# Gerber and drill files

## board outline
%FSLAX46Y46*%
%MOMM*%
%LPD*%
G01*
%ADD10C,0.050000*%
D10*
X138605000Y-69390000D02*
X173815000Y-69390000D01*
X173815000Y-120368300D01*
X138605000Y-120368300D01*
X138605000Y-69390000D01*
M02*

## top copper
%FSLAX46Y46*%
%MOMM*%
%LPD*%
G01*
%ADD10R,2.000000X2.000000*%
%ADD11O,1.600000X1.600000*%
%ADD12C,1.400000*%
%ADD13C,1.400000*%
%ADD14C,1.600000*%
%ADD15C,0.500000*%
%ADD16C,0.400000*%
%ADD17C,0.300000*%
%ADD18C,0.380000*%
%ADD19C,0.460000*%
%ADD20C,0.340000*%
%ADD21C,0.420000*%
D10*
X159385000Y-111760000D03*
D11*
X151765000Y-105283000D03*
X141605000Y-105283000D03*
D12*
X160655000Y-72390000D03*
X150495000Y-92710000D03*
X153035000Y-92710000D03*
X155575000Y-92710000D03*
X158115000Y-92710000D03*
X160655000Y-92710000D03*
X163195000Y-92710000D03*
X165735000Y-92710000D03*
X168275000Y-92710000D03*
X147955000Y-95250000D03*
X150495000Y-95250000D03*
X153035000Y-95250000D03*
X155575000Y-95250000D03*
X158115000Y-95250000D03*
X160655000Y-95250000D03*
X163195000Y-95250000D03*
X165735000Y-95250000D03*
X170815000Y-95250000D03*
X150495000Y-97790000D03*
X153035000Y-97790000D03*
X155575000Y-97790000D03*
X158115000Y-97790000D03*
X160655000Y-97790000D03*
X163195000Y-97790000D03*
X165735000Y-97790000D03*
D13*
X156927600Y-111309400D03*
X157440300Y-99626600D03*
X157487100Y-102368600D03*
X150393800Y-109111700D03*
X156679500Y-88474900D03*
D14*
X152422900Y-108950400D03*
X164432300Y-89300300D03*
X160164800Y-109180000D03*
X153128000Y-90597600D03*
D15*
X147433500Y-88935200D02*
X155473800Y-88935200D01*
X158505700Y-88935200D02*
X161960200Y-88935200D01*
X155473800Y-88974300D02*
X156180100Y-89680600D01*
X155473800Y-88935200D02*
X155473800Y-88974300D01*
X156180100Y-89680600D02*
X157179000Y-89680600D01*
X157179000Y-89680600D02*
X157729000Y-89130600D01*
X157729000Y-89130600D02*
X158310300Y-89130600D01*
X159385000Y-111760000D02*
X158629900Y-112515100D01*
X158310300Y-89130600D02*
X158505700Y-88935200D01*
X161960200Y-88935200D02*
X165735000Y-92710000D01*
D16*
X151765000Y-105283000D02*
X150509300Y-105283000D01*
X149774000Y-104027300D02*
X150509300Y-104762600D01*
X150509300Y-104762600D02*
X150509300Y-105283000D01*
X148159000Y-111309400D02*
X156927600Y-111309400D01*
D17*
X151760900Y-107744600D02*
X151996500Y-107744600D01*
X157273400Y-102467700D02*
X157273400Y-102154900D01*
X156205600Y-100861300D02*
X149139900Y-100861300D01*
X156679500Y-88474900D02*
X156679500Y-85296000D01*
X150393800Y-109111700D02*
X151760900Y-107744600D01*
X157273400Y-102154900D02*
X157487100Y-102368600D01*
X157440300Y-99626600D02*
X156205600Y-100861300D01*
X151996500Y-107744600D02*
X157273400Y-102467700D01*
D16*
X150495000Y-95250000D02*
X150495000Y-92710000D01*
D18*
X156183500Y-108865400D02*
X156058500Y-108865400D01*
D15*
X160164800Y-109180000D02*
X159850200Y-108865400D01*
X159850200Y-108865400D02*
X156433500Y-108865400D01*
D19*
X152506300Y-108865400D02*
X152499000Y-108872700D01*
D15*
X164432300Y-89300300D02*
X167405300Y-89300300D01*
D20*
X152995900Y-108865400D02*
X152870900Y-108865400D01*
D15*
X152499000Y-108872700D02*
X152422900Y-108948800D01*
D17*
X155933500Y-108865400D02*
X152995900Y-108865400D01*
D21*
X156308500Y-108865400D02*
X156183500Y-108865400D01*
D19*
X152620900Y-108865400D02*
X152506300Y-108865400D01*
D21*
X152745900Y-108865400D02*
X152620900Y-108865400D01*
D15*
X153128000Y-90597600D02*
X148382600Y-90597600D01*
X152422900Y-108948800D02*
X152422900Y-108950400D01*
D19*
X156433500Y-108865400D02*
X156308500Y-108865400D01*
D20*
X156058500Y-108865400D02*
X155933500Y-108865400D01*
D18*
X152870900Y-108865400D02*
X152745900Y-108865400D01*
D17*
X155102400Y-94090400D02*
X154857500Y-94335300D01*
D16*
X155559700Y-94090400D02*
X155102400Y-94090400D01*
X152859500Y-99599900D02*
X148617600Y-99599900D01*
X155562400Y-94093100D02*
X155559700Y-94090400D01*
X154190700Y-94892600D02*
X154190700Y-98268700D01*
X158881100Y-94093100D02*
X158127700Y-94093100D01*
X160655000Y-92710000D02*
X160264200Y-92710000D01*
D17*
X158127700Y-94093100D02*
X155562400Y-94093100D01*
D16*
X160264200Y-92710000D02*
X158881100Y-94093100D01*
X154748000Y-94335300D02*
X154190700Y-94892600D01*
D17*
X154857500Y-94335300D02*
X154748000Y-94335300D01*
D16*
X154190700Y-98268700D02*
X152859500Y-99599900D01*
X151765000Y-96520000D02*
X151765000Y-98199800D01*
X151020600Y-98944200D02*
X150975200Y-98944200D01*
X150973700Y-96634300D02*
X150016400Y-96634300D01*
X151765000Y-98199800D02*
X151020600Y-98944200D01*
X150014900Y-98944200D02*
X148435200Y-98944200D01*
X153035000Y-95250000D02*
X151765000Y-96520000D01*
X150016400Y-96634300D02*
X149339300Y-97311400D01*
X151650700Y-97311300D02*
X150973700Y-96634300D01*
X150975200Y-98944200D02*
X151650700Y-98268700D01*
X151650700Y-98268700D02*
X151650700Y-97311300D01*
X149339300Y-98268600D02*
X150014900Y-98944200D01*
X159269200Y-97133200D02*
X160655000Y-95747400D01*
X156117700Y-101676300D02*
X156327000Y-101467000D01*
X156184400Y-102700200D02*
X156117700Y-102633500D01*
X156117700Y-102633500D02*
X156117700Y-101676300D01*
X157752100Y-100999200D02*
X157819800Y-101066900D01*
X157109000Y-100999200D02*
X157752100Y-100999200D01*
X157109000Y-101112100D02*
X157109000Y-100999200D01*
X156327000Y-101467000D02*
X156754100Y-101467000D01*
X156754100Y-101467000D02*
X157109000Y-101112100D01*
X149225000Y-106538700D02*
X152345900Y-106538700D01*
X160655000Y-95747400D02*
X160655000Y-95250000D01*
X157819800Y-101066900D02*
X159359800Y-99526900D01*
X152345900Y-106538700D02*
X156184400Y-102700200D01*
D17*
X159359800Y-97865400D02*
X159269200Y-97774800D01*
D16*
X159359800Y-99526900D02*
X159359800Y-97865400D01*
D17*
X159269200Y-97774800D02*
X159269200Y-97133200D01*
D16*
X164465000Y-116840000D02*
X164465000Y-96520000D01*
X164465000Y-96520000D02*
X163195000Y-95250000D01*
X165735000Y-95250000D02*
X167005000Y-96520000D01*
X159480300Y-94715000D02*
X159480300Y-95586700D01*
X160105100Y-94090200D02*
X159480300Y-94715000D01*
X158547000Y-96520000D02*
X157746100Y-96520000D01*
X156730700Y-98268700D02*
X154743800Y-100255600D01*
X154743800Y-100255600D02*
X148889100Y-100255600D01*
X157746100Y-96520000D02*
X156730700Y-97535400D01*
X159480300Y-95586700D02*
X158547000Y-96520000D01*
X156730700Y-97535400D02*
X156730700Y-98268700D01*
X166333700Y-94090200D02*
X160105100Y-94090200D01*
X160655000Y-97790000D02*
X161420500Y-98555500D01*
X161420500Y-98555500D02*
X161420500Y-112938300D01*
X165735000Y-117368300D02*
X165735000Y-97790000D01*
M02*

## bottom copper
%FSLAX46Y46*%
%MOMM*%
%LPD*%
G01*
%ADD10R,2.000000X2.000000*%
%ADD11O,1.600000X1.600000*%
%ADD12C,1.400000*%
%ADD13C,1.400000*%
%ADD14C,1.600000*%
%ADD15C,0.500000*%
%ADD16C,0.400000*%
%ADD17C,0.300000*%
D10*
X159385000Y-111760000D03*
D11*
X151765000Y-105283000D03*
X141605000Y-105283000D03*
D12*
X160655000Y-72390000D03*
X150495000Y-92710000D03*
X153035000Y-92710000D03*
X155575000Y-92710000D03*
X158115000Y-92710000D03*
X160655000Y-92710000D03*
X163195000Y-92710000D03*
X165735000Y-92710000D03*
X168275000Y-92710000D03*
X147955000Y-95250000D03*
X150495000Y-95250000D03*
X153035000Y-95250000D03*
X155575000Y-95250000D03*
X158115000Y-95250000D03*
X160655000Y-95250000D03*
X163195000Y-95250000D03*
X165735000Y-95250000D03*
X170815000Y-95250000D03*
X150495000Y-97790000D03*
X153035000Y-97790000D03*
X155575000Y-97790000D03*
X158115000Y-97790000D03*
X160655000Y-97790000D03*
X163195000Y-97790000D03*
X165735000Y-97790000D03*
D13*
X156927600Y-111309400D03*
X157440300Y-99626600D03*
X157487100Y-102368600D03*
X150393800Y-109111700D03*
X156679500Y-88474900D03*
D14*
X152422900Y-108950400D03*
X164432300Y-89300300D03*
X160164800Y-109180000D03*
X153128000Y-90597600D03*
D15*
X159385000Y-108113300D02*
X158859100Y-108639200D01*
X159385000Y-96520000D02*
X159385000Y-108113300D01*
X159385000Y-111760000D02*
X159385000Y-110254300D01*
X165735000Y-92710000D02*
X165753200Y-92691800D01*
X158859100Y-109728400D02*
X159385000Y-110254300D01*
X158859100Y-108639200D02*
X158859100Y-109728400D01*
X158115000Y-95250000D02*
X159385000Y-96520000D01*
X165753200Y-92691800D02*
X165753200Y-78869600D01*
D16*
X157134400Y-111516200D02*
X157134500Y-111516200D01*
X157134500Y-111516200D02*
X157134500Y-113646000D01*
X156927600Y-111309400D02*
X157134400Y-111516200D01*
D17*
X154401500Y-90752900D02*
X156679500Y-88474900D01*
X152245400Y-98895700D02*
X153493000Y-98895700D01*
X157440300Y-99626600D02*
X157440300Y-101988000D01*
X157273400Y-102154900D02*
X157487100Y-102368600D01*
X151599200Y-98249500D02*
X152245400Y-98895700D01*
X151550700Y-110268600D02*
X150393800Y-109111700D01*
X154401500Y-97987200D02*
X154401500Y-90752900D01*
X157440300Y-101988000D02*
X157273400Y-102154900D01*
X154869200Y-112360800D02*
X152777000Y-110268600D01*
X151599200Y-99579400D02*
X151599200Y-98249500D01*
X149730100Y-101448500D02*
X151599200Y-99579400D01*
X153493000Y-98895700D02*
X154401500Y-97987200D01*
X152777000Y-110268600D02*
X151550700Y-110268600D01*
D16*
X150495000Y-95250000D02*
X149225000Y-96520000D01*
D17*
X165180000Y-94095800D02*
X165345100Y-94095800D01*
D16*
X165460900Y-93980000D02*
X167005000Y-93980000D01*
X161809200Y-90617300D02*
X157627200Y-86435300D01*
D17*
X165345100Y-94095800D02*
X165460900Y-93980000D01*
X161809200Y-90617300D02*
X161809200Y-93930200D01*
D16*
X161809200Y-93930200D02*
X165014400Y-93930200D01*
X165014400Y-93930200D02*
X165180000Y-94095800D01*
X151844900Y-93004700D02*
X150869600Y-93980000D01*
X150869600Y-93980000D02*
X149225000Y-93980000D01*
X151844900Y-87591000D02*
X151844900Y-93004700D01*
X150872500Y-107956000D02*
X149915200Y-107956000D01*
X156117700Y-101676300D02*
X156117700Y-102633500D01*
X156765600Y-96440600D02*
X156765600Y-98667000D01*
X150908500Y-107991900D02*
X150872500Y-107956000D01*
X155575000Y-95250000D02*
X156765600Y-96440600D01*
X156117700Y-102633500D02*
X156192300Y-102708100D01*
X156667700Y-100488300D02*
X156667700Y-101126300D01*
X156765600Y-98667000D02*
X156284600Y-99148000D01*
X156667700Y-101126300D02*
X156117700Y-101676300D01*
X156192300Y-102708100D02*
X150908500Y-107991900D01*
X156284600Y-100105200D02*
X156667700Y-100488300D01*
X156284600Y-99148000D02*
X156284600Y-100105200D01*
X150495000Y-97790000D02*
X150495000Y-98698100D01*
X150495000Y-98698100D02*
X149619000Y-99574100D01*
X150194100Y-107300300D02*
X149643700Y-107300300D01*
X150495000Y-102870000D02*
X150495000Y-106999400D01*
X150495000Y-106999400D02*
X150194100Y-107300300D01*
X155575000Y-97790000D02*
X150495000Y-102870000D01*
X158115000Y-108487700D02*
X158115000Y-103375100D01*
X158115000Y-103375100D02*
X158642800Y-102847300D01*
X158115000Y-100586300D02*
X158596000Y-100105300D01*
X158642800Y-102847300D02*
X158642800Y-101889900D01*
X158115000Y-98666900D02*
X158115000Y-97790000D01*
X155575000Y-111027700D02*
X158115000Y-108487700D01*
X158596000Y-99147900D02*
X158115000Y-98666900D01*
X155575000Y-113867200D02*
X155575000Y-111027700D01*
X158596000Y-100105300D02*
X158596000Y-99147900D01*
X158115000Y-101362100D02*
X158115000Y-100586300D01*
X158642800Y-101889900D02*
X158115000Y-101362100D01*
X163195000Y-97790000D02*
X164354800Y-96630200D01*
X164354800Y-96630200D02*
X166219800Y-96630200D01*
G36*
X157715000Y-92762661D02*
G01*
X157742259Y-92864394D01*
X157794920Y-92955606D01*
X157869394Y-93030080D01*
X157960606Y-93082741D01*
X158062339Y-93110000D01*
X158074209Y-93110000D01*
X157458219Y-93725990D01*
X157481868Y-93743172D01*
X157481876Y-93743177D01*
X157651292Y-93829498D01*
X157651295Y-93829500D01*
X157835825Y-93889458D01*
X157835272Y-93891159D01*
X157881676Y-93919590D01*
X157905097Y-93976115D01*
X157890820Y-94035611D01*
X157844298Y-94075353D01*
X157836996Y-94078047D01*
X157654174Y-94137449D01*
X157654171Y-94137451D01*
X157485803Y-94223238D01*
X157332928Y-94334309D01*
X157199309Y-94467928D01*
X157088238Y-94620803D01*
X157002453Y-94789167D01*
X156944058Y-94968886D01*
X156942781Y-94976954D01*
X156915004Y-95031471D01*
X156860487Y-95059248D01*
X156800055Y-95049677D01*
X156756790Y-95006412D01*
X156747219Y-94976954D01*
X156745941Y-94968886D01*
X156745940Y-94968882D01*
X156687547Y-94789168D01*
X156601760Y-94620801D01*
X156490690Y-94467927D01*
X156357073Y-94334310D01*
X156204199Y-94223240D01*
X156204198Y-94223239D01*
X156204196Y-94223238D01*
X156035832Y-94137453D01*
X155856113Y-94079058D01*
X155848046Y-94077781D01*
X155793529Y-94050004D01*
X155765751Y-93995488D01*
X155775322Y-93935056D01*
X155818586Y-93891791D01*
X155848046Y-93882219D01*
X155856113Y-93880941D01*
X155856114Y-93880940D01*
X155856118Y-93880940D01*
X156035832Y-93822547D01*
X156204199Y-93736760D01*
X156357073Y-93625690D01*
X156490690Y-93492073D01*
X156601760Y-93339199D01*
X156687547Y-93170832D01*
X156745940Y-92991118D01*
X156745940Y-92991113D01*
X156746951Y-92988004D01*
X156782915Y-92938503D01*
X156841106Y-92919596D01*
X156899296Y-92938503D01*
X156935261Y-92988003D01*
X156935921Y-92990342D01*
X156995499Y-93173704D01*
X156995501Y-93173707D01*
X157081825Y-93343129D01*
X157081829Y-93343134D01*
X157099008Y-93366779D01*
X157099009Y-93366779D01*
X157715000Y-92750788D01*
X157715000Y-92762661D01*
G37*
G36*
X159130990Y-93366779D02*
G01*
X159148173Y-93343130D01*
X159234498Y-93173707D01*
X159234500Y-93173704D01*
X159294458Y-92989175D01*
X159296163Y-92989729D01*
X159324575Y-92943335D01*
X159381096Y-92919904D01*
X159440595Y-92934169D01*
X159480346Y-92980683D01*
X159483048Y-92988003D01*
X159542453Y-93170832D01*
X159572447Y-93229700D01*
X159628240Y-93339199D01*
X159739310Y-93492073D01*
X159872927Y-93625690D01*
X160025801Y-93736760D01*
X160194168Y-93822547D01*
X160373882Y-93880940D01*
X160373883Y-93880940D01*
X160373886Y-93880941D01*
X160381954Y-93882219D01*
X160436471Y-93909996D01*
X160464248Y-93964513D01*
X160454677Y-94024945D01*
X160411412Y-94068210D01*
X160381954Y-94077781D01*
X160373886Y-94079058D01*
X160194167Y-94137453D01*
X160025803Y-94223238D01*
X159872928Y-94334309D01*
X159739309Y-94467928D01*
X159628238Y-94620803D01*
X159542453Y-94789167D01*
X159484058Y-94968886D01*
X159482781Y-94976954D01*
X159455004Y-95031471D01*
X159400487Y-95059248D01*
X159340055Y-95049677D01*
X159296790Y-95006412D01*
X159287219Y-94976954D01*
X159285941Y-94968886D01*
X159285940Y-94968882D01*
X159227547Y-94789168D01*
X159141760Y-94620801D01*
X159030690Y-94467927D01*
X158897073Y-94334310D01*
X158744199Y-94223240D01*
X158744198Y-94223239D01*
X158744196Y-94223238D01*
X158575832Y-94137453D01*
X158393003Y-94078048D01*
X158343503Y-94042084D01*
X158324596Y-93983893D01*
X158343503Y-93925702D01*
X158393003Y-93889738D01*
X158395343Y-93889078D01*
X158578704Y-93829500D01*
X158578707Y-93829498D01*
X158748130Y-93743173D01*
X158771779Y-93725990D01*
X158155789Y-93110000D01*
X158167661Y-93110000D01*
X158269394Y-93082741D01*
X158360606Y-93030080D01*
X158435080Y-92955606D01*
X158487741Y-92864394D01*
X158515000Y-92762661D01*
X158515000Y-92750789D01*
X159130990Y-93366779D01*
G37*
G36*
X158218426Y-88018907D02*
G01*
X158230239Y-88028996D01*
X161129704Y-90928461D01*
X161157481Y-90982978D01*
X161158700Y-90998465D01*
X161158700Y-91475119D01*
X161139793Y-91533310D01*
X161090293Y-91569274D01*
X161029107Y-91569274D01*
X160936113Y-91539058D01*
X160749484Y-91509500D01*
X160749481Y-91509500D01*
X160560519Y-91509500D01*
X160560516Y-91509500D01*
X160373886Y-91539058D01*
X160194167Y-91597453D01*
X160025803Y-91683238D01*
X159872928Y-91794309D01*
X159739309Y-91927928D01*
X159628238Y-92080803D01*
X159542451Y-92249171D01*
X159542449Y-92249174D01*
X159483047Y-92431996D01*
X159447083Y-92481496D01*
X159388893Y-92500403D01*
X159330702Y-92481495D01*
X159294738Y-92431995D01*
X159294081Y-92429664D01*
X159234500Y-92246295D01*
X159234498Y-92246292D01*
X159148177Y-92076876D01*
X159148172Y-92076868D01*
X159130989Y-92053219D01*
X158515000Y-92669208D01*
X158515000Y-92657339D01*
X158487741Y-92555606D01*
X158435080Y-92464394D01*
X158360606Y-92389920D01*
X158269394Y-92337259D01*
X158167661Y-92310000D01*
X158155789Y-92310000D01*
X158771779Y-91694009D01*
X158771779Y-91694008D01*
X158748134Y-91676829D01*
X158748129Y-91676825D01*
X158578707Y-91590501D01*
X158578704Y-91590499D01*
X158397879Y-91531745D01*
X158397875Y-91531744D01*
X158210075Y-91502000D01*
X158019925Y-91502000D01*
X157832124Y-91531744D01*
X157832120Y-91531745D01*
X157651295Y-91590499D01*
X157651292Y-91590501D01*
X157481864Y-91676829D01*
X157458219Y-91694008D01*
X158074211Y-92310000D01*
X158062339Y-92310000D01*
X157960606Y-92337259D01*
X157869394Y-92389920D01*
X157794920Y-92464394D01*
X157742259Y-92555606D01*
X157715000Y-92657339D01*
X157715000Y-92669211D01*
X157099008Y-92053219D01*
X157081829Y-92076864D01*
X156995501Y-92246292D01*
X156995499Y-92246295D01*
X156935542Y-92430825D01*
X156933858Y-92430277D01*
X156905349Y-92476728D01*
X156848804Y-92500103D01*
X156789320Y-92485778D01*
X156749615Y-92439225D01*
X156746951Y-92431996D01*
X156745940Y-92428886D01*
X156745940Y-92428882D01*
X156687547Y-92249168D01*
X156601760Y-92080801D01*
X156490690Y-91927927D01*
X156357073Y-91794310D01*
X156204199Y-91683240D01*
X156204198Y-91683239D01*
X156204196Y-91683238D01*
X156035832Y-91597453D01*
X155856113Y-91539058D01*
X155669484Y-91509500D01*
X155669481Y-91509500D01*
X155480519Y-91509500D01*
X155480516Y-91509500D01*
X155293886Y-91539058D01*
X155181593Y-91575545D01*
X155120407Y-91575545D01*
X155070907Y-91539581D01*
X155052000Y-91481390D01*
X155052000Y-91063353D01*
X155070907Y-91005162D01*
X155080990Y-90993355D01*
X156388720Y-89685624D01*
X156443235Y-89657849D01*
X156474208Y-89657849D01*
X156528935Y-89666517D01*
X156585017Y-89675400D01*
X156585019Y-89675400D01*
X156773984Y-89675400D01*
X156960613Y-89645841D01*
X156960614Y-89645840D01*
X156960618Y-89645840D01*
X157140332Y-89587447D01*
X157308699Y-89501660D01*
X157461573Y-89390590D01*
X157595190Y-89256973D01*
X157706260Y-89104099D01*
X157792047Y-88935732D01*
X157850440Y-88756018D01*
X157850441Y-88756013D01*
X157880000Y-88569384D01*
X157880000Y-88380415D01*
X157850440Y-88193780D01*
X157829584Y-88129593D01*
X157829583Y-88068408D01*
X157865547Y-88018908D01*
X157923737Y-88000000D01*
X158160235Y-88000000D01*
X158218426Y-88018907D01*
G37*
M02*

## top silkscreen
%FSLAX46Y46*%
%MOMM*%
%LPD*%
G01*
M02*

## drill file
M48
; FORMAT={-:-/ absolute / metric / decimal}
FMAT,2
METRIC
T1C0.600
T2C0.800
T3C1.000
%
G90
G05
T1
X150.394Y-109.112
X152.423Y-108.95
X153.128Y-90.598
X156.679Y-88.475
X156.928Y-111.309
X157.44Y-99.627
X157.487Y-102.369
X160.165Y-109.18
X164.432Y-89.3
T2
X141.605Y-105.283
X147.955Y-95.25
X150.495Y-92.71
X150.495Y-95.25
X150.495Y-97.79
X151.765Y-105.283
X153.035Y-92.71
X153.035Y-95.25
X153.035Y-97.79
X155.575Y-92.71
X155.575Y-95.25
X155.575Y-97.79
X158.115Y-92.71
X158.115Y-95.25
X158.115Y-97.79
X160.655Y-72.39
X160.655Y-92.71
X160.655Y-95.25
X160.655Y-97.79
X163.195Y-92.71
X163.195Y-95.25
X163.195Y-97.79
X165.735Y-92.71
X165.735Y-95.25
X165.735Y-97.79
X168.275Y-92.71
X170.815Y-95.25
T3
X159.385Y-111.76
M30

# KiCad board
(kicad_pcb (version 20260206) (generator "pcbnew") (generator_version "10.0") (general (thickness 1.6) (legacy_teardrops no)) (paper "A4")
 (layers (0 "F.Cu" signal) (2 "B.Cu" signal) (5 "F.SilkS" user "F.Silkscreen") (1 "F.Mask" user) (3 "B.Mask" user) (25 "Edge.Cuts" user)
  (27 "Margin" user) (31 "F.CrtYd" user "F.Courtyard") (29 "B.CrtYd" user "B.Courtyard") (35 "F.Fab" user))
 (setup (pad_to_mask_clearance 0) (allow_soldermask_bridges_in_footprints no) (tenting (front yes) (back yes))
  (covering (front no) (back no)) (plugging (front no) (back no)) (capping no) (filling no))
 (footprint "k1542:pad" (layer "F.Cu") (at 159.385 111.76)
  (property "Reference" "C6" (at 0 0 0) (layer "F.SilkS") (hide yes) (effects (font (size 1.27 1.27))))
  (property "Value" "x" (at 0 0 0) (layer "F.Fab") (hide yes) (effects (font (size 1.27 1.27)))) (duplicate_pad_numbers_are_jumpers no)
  (pad "1" thru_hole rect (at 0 0) (size 2 2) (drill 1) (layers "*.Cu" "*.Mask") (remove_unused_layers no) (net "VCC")))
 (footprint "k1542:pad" (layer "F.Cu") (at 151.765 105.283 90)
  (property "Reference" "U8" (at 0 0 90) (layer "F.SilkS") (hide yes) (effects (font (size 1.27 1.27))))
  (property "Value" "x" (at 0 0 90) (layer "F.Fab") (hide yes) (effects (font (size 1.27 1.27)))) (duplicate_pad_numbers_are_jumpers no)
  (pad "13" thru_hole oval (at 0 0 90) (size 1.6 1.6) (drill 0.8) (layers "*.Cu" "*.Mask") (remove_unused_layers no) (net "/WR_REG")))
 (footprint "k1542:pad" (layer "F.Cu") (at 141.605 105.283 90)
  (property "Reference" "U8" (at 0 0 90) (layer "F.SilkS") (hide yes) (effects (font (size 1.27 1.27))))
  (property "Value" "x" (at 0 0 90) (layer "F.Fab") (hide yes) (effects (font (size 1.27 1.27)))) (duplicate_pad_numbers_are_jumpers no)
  (pad "17" thru_hole oval (at 0 0 90) (size 1.6 1.6) (drill 0.8) (layers "*.Cu" "*.Mask") (remove_unused_layers no) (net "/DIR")))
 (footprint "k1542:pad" (layer "F.Cu") (at 160.655 72.39 180)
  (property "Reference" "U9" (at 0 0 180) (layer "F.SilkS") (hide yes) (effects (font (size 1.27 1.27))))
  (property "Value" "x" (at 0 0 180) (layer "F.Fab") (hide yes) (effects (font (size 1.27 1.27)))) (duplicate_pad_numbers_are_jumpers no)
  (pad "C8" thru_hole circle (at 0 0 180) (size 1.4 1.4) (drill 0.8) (layers "*.Cu" "*.Mask") (remove_unused_layers no) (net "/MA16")))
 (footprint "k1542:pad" (layer "F.Cu") (at 150.495 92.71 180)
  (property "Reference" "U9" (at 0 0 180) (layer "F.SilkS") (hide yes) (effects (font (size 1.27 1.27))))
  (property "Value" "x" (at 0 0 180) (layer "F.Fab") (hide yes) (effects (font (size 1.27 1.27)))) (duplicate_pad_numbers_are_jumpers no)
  (pad "L4" thru_hole circle (at 0 0 180) (size 1.4 1.4) (drill 0.8) (layers "*.Cu" "*.Mask") (remove_unused_layers no) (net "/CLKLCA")))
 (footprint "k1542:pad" (layer "F.Cu") (at 153.035 92.71 180)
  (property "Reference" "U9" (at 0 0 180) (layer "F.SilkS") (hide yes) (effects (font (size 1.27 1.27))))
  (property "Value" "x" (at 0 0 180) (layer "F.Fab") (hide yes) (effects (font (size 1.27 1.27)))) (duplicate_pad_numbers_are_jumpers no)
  (pad "L5" thru_hole circle (at 0 0 180) (size 1.4 1.4) (drill 0.8) (layers "*.Cu" "*.Mask") (remove_unused_layers no)
   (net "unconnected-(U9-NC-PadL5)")))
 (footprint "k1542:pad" (layer "F.Cu") (at 155.575 92.71 180)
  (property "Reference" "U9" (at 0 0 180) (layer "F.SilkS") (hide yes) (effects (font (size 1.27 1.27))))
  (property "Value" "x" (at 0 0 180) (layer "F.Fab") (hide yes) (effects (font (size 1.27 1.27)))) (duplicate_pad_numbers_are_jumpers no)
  (pad "L6" thru_hole circle (at 0 0 180) (size 1.4 1.4) (drill 0.8) (layers "*.Cu" "*.Mask") (remove_unused_layers no)
   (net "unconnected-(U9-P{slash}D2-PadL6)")))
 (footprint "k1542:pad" (layer "F.Cu") (at 158.115 92.71 180)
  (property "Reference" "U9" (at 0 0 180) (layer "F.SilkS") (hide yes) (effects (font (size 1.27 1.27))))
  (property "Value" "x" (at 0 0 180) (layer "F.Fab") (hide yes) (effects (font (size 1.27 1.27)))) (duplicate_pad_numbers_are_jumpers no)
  (pad "L7" thru_hole circle (at 0 0 180) (size 1.4 1.4) (drill 0.8) (layers "*.Cu" "*.Mask") (remove_unused_layers no) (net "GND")))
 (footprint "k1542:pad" (layer "F.Cu") (at 160.655 92.71 180)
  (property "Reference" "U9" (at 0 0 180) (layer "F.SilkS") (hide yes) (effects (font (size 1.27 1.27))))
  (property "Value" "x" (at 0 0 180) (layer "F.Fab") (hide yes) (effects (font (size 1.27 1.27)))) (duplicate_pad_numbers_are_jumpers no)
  (pad "L8" thru_hole circle (at 0 0 180) (size 1.4 1.4) (drill 0.8) (layers "*.Cu" "*.Mask") (remove_unused_layers no) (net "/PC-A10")))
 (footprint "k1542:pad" (layer "F.Cu") (at 163.195 92.71 180)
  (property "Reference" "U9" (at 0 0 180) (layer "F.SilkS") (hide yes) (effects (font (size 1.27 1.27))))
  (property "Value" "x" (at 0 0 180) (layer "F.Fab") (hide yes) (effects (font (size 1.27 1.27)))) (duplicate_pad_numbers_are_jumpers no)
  (pad "L9" thru_hole circle (at 0 0 180) (size 1.4 1.4) (drill 0.8) (layers "*.Cu" "*.Mask") (remove_unused_layers no)
   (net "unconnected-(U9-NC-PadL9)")))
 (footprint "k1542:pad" (layer "F.Cu") (at 165.735 92.71 180)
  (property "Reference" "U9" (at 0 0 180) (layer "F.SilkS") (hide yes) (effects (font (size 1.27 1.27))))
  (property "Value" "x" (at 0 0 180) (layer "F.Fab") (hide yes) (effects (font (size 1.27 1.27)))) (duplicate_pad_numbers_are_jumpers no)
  (pad "L10" thru_hole circle (at 0 0 180) (size 1.4 1.4) (drill 0.8) (layers "*.Cu" "*.Mask") (remove_unused_layers no) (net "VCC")))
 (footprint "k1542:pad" (layer "F.Cu") (at 168.275 92.71 180)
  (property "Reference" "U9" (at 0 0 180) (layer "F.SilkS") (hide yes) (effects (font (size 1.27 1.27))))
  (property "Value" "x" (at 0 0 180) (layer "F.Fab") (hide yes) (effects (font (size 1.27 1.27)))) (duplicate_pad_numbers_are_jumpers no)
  (pad "L11" thru_hole circle (at 0 0 180) (size 1.4 1.4) (drill 0.8) (layers "*.Cu" "*.Mask") (remove_unused_layers no) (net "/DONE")))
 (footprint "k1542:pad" (layer "F.Cu") (at 147.955 95.25 180)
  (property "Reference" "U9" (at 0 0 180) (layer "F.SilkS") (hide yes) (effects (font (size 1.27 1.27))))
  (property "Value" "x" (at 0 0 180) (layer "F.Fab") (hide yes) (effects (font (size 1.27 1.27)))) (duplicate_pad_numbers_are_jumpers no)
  (pad "M3" thru_hole circle (at 0 0 180) (size 1.4 1.4) (drill 0.8) (layers "*.Cu" "*.Mask") (remove_unused_layers no) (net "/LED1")))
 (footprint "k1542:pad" (layer "F.Cu") (at 150.495 95.25 180)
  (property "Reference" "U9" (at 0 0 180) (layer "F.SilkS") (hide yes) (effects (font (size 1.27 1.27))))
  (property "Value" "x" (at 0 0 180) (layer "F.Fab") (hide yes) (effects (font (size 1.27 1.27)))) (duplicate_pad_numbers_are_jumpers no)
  (pad "M4" thru_hole circle (at 0 0 180) (size 1.4 1.4) (drill 0.8) (layers "*.Cu" "*.Mask") (remove_unused_layers no) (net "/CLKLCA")))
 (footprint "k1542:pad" (layer "F.Cu") (at 153.035 95.25 180)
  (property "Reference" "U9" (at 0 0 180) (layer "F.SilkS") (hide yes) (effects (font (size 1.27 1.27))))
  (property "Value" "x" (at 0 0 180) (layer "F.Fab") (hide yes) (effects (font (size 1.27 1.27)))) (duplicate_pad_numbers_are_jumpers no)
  (pad "M5" thru_hole circle (at 0 0 180) (size 1.4 1.4) (drill 0.8) (layers "*.Cu" "*.Mask") (remove_unused_layers no) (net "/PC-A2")))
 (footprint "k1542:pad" (layer "F.Cu") (at 155.575 95.25 180)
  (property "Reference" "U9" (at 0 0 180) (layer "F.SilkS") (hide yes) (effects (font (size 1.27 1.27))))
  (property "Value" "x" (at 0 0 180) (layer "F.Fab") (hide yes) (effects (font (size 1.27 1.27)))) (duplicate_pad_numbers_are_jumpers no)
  (pad "M6" thru_hole circle (at 0 0 180) (size 1.4 1.4) (drill 0.8) (layers "*.Cu" "*.Mask") (remove_unused_layers no) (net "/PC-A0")))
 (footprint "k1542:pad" (layer "F.Cu") (at 158.115 95.25 180)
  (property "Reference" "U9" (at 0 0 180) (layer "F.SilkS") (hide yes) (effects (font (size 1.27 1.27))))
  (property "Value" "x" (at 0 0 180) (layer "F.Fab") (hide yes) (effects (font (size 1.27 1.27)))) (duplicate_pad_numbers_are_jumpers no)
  (pad "M7" thru_hole circle (at 0 0 180) (size 1.4 1.4) (drill 0.8) (layers "*.Cu" "*.Mask") (remove_unused_layers no) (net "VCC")))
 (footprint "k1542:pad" (layer "F.Cu") (at 160.655 95.25 180)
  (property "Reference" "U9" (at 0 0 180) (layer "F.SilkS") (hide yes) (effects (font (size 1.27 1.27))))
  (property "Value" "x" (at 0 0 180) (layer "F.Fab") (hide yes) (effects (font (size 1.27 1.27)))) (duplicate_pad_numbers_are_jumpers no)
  (pad "M8" thru_hole circle (at 0 0 180) (size 1.4 1.4) (drill 0.8) (layers "*.Cu" "*.Mask") (remove_unused_layers no) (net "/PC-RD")))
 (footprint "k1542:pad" (layer "F.Cu") (at 163.195 95.25 180)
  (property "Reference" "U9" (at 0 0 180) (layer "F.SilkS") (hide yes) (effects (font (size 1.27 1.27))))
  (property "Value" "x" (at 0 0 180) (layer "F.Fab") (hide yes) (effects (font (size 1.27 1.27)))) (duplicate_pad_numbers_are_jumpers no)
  (pad "M9" thru_hole circle (at 0 0 180) (size 1.4 1.4) (drill 0.8) (layers "*.Cu" "*.Mask") (remove_unused_layers no) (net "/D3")))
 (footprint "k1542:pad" (layer "F.Cu") (at 165.735 95.25 180)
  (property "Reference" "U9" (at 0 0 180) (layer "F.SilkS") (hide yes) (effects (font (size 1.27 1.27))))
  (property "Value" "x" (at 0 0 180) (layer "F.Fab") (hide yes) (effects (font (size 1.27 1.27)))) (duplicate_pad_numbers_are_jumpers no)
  (pad "M10" thru_hole circle (at 0 0 180) (size 1.4 1.4) (drill 0.8) (layers "*.Cu" "*.Mask") (remove_unused_layers no) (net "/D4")))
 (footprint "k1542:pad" (layer "F.Cu") (at 170.815 95.25 180)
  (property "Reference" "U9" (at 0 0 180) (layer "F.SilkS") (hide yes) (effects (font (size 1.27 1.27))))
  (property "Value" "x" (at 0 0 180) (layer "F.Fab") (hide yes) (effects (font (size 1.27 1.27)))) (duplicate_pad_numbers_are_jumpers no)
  (pad "M12" thru_hole circle (at 0 0 180) (size 1.4 1.4) (drill 0.8) (layers "*.Cu" "*.Mask") (remove_unused_layers no) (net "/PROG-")))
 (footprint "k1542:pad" (layer "F.Cu") (at 150.495 97.79 180)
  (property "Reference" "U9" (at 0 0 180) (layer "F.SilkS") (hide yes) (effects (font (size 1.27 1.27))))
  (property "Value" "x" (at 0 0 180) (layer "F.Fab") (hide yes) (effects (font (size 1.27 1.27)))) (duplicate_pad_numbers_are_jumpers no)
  (pad "N4" thru_hole circle (at 0 0 180) (size 1.4 1.4) (drill 0.8) (layers "*.Cu" "*.Mask") (remove_unused_layers no) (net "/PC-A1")))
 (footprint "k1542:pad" (layer "F.Cu") (at 153.035 97.79 180)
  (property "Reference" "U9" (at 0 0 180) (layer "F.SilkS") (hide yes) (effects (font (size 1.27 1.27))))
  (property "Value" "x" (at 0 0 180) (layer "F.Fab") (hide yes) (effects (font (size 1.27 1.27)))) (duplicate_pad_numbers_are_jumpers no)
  (pad "N5" thru_hole circle (at 0 0 180) (size 1.4 1.4) (drill 0.8) (layers "*.Cu" "*.Mask") (remove_unused_layers no)
   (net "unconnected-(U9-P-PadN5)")))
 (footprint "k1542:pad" (layer "F.Cu") (at 155.575 97.79 180)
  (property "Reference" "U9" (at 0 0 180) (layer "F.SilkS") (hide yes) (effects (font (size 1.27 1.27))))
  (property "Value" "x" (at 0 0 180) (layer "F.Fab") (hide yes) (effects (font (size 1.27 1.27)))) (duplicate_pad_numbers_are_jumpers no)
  (pad "N6" thru_hole circle (at 0 0 180) (size 1.4 1.4) (drill 0.8) (layers "*.Cu" "*.Mask") (remove_unused_layers no) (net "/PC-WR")))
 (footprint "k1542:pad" (layer "F.Cu") (at 158.115 97.79 180)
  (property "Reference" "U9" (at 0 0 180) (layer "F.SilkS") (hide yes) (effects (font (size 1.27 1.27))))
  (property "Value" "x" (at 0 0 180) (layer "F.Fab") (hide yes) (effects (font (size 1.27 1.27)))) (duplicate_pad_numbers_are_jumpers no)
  (pad "N7" thru_hole circle (at 0 0 180) (size 1.4 1.4) (drill 0.8) (layers "*.Cu" "*.Mask") (remove_unused_layers no) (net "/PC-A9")))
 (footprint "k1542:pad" (layer "F.Cu") (at 160.655 97.79 180)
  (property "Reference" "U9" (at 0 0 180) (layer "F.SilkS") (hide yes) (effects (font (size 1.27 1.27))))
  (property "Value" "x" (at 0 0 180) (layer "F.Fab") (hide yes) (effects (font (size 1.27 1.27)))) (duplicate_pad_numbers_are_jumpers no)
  (pad "N8" thru_hole circle (at 0 0 180) (size 1.4 1.4) (drill 0.8) (layers "*.Cu" "*.Mask") (remove_unused_layers no) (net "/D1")))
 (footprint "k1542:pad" (layer "F.Cu") (at 163.195 97.79 180)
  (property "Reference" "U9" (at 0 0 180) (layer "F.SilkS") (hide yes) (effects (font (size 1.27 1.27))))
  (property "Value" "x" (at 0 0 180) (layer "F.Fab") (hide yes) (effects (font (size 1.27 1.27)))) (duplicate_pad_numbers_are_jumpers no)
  (pad "N9" thru_hole circle (at 0 0 180) (size 1.4 1.4) (drill 0.8) (layers "*.Cu" "*.Mask") (remove_unused_layers no) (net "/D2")))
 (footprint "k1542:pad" (layer "F.Cu") (at 165.735 97.79 180)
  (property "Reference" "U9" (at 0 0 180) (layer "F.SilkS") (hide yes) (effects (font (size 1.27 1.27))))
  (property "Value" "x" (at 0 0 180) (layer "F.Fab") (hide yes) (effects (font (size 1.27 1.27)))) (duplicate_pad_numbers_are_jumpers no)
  (pad "N10" thru_hole circle (at 0 0 180) (size 1.4 1.4) (drill 0.8) (layers "*.Cu" "*.Mask") (remove_unused_layers no) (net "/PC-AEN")))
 (gr_rect (start 138.605 69.39) (end 173.815 120.3683) (stroke (width 0.05) (type default)) (fill no) (layer "Edge.Cuts"))
 (segment (start 147.4335 88.9352) (end 155.4738 88.9352) (width 0.5) (layer "F.Cu") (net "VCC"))
 (segment (start 158.5057 88.9352) (end 161.9602 88.9352) (width 0.5) (layer "F.Cu") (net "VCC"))
 (segment (start 155.4738 88.9743) (end 156.1801 89.6806) (width 0.5) (layer "F.Cu") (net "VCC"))
 (segment (start 155.4738 88.9352) (end 155.4738 88.9743) (width 0.5) (layer "F.Cu") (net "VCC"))
 (segment (start 156.1801 89.6806) (end 157.179 89.6806) (width 0.5) (layer "F.Cu") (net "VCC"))
 (segment (start 157.179 89.6806) (end 157.729 89.1306) (width 0.5) (layer "F.Cu") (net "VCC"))
 (segment (start 157.729 89.1306) (end 158.3103 89.1306) (width 0.5) (layer "F.Cu") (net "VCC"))
 (segment (start 159.385 111.76) (end 158.6299 112.5151) (width 0.5) (layer "F.Cu") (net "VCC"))
 (segment (start 158.3103 89.1306) (end 158.5057 88.9352) (width 0.5) (layer "F.Cu") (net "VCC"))
 (segment (start 161.9602 88.9352) (end 165.735 92.71) (width 0.5) (layer "F.Cu") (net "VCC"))
 (segment (start 159.385 108.1133) (end 158.8591 108.6392) (width 0.5) (layer "B.Cu") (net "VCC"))
 (segment (start 159.385 96.52) (end 159.385 108.1133) (width 0.5) (layer "B.Cu") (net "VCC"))
 (segment (start 159.385 111.76) (end 159.385 110.2543) (width 0.5) (layer "B.Cu") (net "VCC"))
 (segment (start 165.735 92.71) (end 165.7532 92.6918) (width 0.5) (layer "B.Cu") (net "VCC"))
 (segment (start 158.8591 109.7284) (end 159.385 110.2543) (width 0.5) (layer "B.Cu") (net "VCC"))
 (segment (start 158.8591 108.6392) (end 158.8591 109.7284) (width 0.5) (layer "B.Cu") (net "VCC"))
 (segment (start 158.115 95.25) (end 159.385 96.52) (width 0.5) (layer "B.Cu") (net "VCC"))
 (segment (start 165.7532 92.6918) (end 165.7532 78.8696) (width 0.5) (layer "B.Cu") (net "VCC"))
 (segment (start 151.765 105.283) (end 150.5093 105.283) (width 0.4) (layer "F.Cu") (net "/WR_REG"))
 (segment (start 149.774 104.0273) (end 150.5093 104.7626) (width 0.4) (layer "F.Cu") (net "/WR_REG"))
 (segment (start 150.5093 104.7626) (end 150.5093 105.283) (width 0.4) (layer "F.Cu") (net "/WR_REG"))
 (segment (start 148.159 111.3094) (end 156.9276 111.3094) (width 0.4) (layer "F.Cu") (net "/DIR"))
 (via (at 156.9276 111.3094) (size 1.4) (drill 0.6) (layers "F.Cu" "B.Cu") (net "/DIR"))
 (segment (start 157.1344 111.5162) (end 157.1345 111.5162) (width 0.4) (layer "B.Cu") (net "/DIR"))
 (segment (start 157.1345 111.5162) (end 157.1345 113.646) (width 0.4) (layer "B.Cu") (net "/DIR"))
 (segment (start 156.9276 111.3094) (end 157.1344 111.5162) (width 0.4) (layer "B.Cu") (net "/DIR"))
 (segment (start 151.7609 107.7446) (end 151.9965 107.7446) (width 0.3) (layer "F.Cu") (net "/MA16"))
 (segment (start 157.2734 102.4677) (end 157.2734 102.1549) (width 0.3) (layer "F.Cu") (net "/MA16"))
 (segment (start 156.2056 100.8613) (end 149.1399 100.8613) (width 0.3) (layer "F.Cu") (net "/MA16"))
 (segment (start 156.6795 88.4749) (end 156.6795 85.296) (width 0.3) (layer "F.Cu") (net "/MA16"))
 (segment (start 150.3938 109.1117) (end 151.7609 107.7446) (width 0.3) (layer "F.Cu") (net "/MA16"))
 (segment (start 157.2734 102.1549) (end 157.4871 102.3686) (width 0.3) (layer "F.Cu") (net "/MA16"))
 (segment (start 157.4403 99.6266) (end 156.2056 100.8613) (width 0.3) (layer "F.Cu") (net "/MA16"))
 (segment (start 151.9965 107.7446) (end 157.2734 102.4677) (width 0.3) (layer "F.Cu") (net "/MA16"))
 (via (at 157.4403 99.6266) (size 1.4) (drill 0.6) (layers "F.Cu" "B.Cu") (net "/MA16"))
 (via (at 157.4871 102.3686) (size 1.4) (drill 0.6) (layers "F.Cu" "B.Cu") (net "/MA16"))
 (via (at 150.3938 109.1117) (size 1.4) (drill 0.6) (layers "F.Cu" "B.Cu") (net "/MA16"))
 (via (at 156.6795 88.4749) (size 1.4) (drill 0.6) (layers "F.Cu" "B.Cu") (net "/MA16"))
 (segment (start 154.4015 90.7529) (end 156.6795 88.4749) (width 0.3) (layer "B.Cu") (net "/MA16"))
 (segment (start 152.2454 98.8957) (end 153.493 98.8957) (width 0.3) (layer "B.Cu") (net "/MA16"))
 (segment (start 157.4403 99.6266) (end 157.4403 101.988) (width 0.3) (layer "B.Cu") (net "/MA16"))
 (segment (start 157.2734 102.1549) (end 157.4871 102.3686) (width 0.3) (layer "B.Cu") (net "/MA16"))
 (segment (start 151.5992 98.2495) (end 152.2454 98.8957) (width 0.3) (layer "B.Cu") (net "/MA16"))
 (segment (start 151.5507 110.2686) (end 150.3938 109.1117) (width 0.3) (layer "B.Cu") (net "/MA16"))
 (segment (start 154.4015 97.9872) (end 154.4015 90.7529) (width 0.3) (layer "B.Cu") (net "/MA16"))
 (segment (start 157.4403 101.988) (end 157.2734 102.1549) (width 0.3) (layer "B.Cu") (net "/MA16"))
 (segment (start 154.8692 112.3608) (end 152.777 110.2686) (width 0.3) (layer "B.Cu") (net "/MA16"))
 (segment (start 151.5992 99.5794) (end 151.5992 98.2495) (width 0.3) (layer "B.Cu") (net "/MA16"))
 (segment (start 149.7301 101.4485) (end 151.5992 99.5794) (width 0.3) (layer "B.Cu") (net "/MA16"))
 (segment (start 153.493 98.8957) (end 154.4015 97.9872) (width 0.3) (layer "B.Cu") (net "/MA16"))
 (segment (start 152.777 110.2686) (end 151.5507 110.2686) (width 0.3) (layer "B.Cu") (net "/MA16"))
 (segment (start 150.495 95.25) (end 150.495 92.71) (width 0.4) (layer "F.Cu") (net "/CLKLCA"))
 (segment (start 150.495 95.25) (end 149.225 96.52) (width 0.4) (layer "B.Cu") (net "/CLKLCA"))
 (segment (start 156.1835 108.8654) (end 156.0585 108.8654) (width 0.38) (layer "F.Cu") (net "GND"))
 (segment (start 160.1648 109.18) (end 159.8502 108.8654) (width 0.5) (layer "F.Cu") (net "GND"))
 (segment (start 159.8502 108.8654) (end 156.4335 108.8654) (width 0.5) (layer "F.Cu") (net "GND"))
 (segment (start 152.5063 108.8654) (end 152.499 108.8727) (width 0.46) (layer "F.Cu") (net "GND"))
 (segment (start 164.4323 89.3003) (end 167.4053 89.3003) (width 0.5) (layer "F.Cu") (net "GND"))
 (segment (start 152.9959 108.8654) (end 152.8709 108.8654) (width 0.34) (layer "F.Cu") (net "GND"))
 (segment (start 152.499 108.8727) (end 152.4229 108.9488) (width 0.5) (layer "F.Cu") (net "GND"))
 (segment (start 155.9335 108.8654) (end 152.9959 108.8654) (width 0.3) (layer "F.Cu") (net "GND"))
 (segment (start 156.3085 108.8654) (end 156.1835 108.8654) (width 0.42) (layer "F.Cu") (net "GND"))
 (segment (start 152.6209 108.8654) (end 152.5063 108.8654) (width 0.46) (layer "F.Cu") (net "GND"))
 (segment (start 152.7459 108.8654) (end 152.6209 108.8654) (width 0.42) (layer "F.Cu") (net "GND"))
 (segment (start 153.128 90.5976) (end 148.3826 90.5976) (width 0.5) (layer "F.Cu") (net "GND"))
 (segment (start 152.4229 108.9488) (end 152.4229 108.9504) (width 0.5) (layer "F.Cu") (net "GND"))
 (segment (start 156.4335 108.8654) (end 156.3085 108.8654) (width 0.46) (layer "F.Cu") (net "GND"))
 (segment (start 156.0585 108.8654) (end 155.9335 108.8654) (width 0.34) (layer "F.Cu") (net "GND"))
 (segment (start 152.8709 108.8654) (end 152.7459 108.8654) (width 0.38) (layer "F.Cu") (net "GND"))
 (via (at 152.4229 108.9504) (size 1.6) (drill 0.6) (layers "F.Cu" "B.Cu") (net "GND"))
 (via (at 164.4323 89.3003) (size 1.6) (drill 0.6) (layers "F.Cu" "B.Cu") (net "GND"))
 (via (at 160.1648 109.18) (size 1.6) (drill 0.6) (layers "F.Cu" "B.Cu") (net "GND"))
 (via (at 153.128 90.5976) (size 1.6) (drill 0.6) (layers "F.Cu" "B.Cu") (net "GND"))
 (segment (start 155.1024 94.0904) (end 154.8575 94.3353) (width 0.3) (layer "F.Cu") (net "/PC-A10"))
 (segment (start 155.5597 94.0904) (end 155.1024 94.0904) (width 0.4) (layer "F.Cu") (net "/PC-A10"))
 (segment (start 152.8595 99.5999) (end 148.6176 99.5999) (width 0.4) (layer "F.Cu") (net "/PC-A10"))
 (segment (start 155.5624 94.0931) (end 155.5597 94.0904) (width 0.4) (layer "F.Cu") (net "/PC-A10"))
 (segment (start 154.1907 94.8926) (end 154.1907 98.2687) (width 0.4) (layer "F.Cu") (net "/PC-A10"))
 (segment (start 158.8811 94.0931) (end 158.1277 94.0931) (width 0.4) (layer "F.Cu") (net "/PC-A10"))
 (segment (start 160.655 92.71) (end 160.2642 92.71) (width 0.4) (layer "F.Cu") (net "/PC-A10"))
 (segment (start 158.1277 94.0931) (end 155.5624 94.0931) (width 0.3) (layer "F.Cu") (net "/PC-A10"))
 (segment (start 160.2642 92.71) (end 158.8811 94.0931) (width 0.4) (layer "F.Cu") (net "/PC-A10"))
 (segment (start 154.748 94.3353) (end 154.1907 94.8926) (width 0.4) (layer "F.Cu") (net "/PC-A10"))
 (segment (start 154.8575 94.3353) (end 154.748 94.3353) (width 0.3) (layer "F.Cu") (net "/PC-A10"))
 (segment (start 154.1907 98.2687) (end 152.8595 99.5999) (width 0.4) (layer "F.Cu") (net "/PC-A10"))
 (segment (start 165.18 94.0958) (end 165.3451 94.0958) (width 0.3) (layer "B.Cu") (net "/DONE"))
 (segment (start 165.4609 93.98) (end 167.005 93.98) (width 0.4) (layer "B.Cu") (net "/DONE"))
 (segment (start 161.8092 90.6173) (end 157.6272 86.4353) (width 0.4) (layer "B.Cu") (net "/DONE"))
 (segment (start 165.3451 94.0958) (end 165.4609 93.98) (width 0.3) (layer "B.Cu") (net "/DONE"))
 (segment (start 161.8092 90.6173) (end 161.8092 93.9302) (width 0.3) (layer "B.Cu") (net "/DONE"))
 (segment (start 161.8092 93.9302) (end 165.0144 93.9302) (width 0.4) (layer "B.Cu") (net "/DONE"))
 (segment (start 165.0144 93.9302) (end 165.18 94.0958) (width 0.4) (layer "B.Cu") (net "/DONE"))
 (segment (start 151.8449 93.0047) (end 150.8696 93.98) (width 0.4) (layer "B.Cu") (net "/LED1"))
 (segment (start 150.8696 93.98) (end 149.225 93.98) (width 0.4) (layer "B.Cu") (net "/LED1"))
 (segment (start 151.8449 87.591) (end 151.8449 93.0047) (width 0.4) (layer "B.Cu") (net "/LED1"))
 (segment (start 151.765 96.52) (end 151.765 98.1998) (width 0.4) (layer "F.Cu") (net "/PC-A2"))
 (segment (start 151.0206 98.9442) (end 150.9752 98.9442) (width 0.4) (layer "F.Cu") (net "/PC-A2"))
 (segment (start 150.9737 96.6343) (end 150.0164 96.6343) (width 0.4) (layer "F.Cu") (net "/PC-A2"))
 (segment (start 151.765 98.1998) (end 151.0206 98.9442) (width 0.4) (layer "F.Cu") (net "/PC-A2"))
 (segment (start 150.0149 98.9442) (end 148.4352 98.9442) (width 0.4) (layer "F.Cu") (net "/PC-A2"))
 (segment (start 153.035 95.25) (end 151.765 96.52) (width 0.4) (layer "F.Cu") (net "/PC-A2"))
 (segment (start 150.0164 96.6343) (end 149.3393 97.3114) (width 0.4) (layer "F.Cu") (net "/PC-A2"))
 (segment (start 151.6507 97.3113) (end 150.9737 96.6343) (width 0.4) (layer "F.Cu") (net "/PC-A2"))
 (segment (start 150.9752 98.9442) (end 151.6507 98.2687) (width 0.4) (layer "F.Cu") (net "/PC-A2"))
 (segment (start 151.6507 98.2687) (end 151.6507 97.3113) (width 0.4) (layer "F.Cu") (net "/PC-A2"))
 (segment (start 149.3393 98.2686) (end 150.0149 98.9442) (width 0.4) (layer "F.Cu") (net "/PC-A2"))
 (segment (start 150.8725 107.956) (end 149.9152 107.956) (width 0.4) (layer "B.Cu") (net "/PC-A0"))
 (segment (start 156.1177 101.6763) (end 156.1177 102.6335) (width 0.4) (layer "B.Cu") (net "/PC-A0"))
 (segment (start 156.7656 96.4406) (end 156.7656 98.667) (width 0.4) (layer "B.Cu") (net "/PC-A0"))
 (segment (start 150.9085 107.9919) (end 150.8725 107.956) (width 0.4) (layer "B.Cu") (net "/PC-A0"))
 (segment (start 155.575 95.25) (end 156.7656 96.4406) (width 0.4) (layer "B.Cu") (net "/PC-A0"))
 (segment (start 156.1177 102.6335) (end 156.1923 102.7081) (width 0.4) (layer "B.Cu") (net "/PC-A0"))
 (segment (start 156.6677 100.4883) (end 156.6677 101.1263) (width 0.4) (layer "B.Cu") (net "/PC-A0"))
 (segment (start 156.7656 98.667) (end 156.2846 99.148) (width 0.4) (layer "B.Cu") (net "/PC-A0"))
 (segment (start 156.6677 101.1263) (end 156.1177 101.6763) (width 0.4) (layer "B.Cu") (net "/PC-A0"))
 (segment (start 156.1923 102.7081) (end 150.9085 107.9919) (width 0.4) (layer "B.Cu") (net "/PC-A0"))
 (segment (start 156.2846 100.1052) (end 156.6677 100.4883) (width 0.4) (layer "B.Cu") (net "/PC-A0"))
 (segment (start 156.2846 99.148) (end 156.2846 100.1052) (width 0.4) (layer "B.Cu") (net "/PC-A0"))
 (segment (start 159.2692 97.1332) (end 160.655 95.7474) (width 0.4) (layer "F.Cu") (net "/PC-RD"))
 (segment (start 156.1177 101.6763) (end 156.327 101.467) (width 0.4) (layer "F.Cu") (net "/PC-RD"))
 (segment (start 156.1844 102.7002) (end 156.1177 102.6335) (width 0.4) (layer "F.Cu") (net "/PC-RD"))
 (segment (start 156.1177 102.6335) (end 156.1177 101.6763) (width 0.4) (layer "F.Cu") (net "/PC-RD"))
 (segment (start 157.7521 100.9992) (end 157.8198 101.0669) (width 0.4) (layer "F.Cu") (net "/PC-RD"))
 (segment (start 157.109 100.9992) (end 157.7521 100.9992) (width 0.4) (layer "F.Cu") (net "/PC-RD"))
 (segment (start 157.109 101.1121) (end 157.109 100.9992) (width 0.4) (layer "F.Cu") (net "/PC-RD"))
 (segment (start 156.327 101.467) (end 156.7541 101.467) (width 0.4) (layer "F.Cu") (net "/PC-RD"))
 (segment (start 156.7541 101.467) (end 157.109 101.1121) (width 0.4) (layer "F.Cu") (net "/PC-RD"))
 (segment (start 149.225 106.5387) (end 152.3459 106.5387) (width 0.4) (layer "F.Cu") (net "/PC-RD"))
 (segment (start 160.655 95.7474) (end 160.655 95.25) (width 0.4) (layer "F.Cu") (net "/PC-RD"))
 (segment (start 157.8198 101.0669) (end 159.3598 99.5269) (width 0.4) (layer "F.Cu") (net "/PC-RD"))
 (segment (start 152.3459 106.5387) (end 156.1844 102.7002) (width 0.4) (layer "F.Cu") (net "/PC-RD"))
 (segment (start 159.3598 97.8654) (end 159.2692 97.7748) (width 0.3) (layer "F.Cu") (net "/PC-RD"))
 (segment (start 159.3598 99.5269) (end 159.3598 97.8654) (width 0.4) (layer "F.Cu") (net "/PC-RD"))
 (segment (start 159.2692 97.7748) (end 159.2692 97.1332) (width 0.3) (layer "F.Cu") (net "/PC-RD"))
 (segment (start 164.465 116.84) (end 164.465 96.52) (width 0.4) (layer "F.Cu") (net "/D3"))
 (segment (start 164.465 96.52) (end 163.195 95.25) (width 0.4) (layer "F.Cu") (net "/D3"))
 (segment (start 165.735 95.25) (end 167.005 96.52) (width 0.4) (layer "F.Cu") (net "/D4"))
 (segment (start 159.4803 94.715) (end 159.4803 95.5867) (width 0.4) (layer "F.Cu") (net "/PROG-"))
 (segment (start 160.1051 94.0902) (end 159.4803 94.715) (width 0.4) (layer "F.Cu") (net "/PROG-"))
 (segment (start 158.547 96.52) (end 157.7461 96.52) (width 0.4) (layer "F.Cu") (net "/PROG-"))
 (segment (start 156.7307 98.2687) (end 154.7438 100.2556) (width 0.4) (layer "F.Cu") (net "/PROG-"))
 (segment (start 154.7438 100.2556) (end 148.8891 100.2556) (width 0.4) (layer "F.Cu") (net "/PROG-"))
 (segment (start 157.7461 96.52) (end 156.7307 97.5354) (width 0.4) (layer "F.Cu") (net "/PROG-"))
 (segment (start 159.4803 95.5867) (end 158.547 96.52) (width 0.4) (layer "F.Cu") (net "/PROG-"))
 (segment (start 156.7307 97.5354) (end 156.7307 98.2687) (width 0.4) (layer "F.Cu") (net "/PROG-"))
 (segment (start 166.3337 94.0902) (end 160.1051 94.0902) (width 0.4) (layer "F.Cu") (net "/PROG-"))
 (segment (start 150.495 97.79) (end 150.495 98.6981) (width 0.4) (layer "B.Cu") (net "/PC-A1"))
 (segment (start 150.495 98.6981) (end 149.619 99.5741) (width 0.4) (layer "B.Cu") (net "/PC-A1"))
 (segment (start 150.1941 107.3003) (end 149.6437 107.3003) (width 0.4) (layer "B.Cu") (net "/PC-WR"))
 (segment (start 150.495 102.87) (end 150.495 106.9994) (width 0.4) (layer "B.Cu") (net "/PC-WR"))
 (segment (start 150.495 106.9994) (end 150.1941 107.3003) (width 0.4) (layer "B.Cu") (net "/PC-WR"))
 (segment (start 155.575 97.79) (end 150.495 102.87) (width 0.4) (layer "B.Cu") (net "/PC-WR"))
 (segment (start 158.115 108.4877) (end 158.115 103.3751) (width 0.4) (layer "B.Cu") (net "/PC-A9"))
 (segment (start 158.115 103.3751) (end 158.6428 102.8473) (width 0.4) (layer "B.Cu") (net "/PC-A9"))
 (segment (start 158.115 100.5863) (end 158.596 100.1053) (width 0.4) (layer "B.Cu") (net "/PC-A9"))
 (segment (start 158.6428 102.8473) (end 158.6428 101.8899) (width 0.4) (layer "B.Cu") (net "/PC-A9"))
 (segment (start 158.115 98.6669) (end 158.115 97.79) (width 0.4) (layer "B.Cu") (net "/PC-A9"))
 (segment (start 155.575 111.0277) (end 158.115 108.4877) (width 0.4) (layer "B.Cu") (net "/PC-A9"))
 (segment (start 158.596 99.1479) (end 158.115 98.6669) (width 0.4) (layer "B.Cu") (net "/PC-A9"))
 (segment (start 155.575 113.8672) (end 155.575 111.0277) (width 0.4) (layer "B.Cu") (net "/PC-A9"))
 (segment (start 158.596 100.1053) (end 158.596 99.1479) (width 0.4) (layer "B.Cu") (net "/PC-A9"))
 (segment (start 158.115 101.3621) (end 158.115 100.5863) (width 0.4) (layer "B.Cu") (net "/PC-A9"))
 (segment (start 158.6428 101.8899) (end 158.115 101.3621) (width 0.4) (layer "B.Cu") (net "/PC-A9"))
 (segment (start 160.655 97.79) (end 161.4205 98.5555) (width 0.4) (layer "F.Cu") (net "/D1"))
 (segment (start 161.4205 98.5555) (end 161.4205 112.9383) (width 0.4) (layer "F.Cu") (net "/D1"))
 (segment (start 163.195 97.79) (end 164.3548 96.6302) (width 0.4) (layer "B.Cu") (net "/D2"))
 (segment (start 164.3548 96.6302) (end 166.2198 96.6302) (width 0.4) (layer "B.Cu") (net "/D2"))
 (segment (start 165.735 117.3683) (end 165.735 97.79) (width 0.4) (layer "F.Cu") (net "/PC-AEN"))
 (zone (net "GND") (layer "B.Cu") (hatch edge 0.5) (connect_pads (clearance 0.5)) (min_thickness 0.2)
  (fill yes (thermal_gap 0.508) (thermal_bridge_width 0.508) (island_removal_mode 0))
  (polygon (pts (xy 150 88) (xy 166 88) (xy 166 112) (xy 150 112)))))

